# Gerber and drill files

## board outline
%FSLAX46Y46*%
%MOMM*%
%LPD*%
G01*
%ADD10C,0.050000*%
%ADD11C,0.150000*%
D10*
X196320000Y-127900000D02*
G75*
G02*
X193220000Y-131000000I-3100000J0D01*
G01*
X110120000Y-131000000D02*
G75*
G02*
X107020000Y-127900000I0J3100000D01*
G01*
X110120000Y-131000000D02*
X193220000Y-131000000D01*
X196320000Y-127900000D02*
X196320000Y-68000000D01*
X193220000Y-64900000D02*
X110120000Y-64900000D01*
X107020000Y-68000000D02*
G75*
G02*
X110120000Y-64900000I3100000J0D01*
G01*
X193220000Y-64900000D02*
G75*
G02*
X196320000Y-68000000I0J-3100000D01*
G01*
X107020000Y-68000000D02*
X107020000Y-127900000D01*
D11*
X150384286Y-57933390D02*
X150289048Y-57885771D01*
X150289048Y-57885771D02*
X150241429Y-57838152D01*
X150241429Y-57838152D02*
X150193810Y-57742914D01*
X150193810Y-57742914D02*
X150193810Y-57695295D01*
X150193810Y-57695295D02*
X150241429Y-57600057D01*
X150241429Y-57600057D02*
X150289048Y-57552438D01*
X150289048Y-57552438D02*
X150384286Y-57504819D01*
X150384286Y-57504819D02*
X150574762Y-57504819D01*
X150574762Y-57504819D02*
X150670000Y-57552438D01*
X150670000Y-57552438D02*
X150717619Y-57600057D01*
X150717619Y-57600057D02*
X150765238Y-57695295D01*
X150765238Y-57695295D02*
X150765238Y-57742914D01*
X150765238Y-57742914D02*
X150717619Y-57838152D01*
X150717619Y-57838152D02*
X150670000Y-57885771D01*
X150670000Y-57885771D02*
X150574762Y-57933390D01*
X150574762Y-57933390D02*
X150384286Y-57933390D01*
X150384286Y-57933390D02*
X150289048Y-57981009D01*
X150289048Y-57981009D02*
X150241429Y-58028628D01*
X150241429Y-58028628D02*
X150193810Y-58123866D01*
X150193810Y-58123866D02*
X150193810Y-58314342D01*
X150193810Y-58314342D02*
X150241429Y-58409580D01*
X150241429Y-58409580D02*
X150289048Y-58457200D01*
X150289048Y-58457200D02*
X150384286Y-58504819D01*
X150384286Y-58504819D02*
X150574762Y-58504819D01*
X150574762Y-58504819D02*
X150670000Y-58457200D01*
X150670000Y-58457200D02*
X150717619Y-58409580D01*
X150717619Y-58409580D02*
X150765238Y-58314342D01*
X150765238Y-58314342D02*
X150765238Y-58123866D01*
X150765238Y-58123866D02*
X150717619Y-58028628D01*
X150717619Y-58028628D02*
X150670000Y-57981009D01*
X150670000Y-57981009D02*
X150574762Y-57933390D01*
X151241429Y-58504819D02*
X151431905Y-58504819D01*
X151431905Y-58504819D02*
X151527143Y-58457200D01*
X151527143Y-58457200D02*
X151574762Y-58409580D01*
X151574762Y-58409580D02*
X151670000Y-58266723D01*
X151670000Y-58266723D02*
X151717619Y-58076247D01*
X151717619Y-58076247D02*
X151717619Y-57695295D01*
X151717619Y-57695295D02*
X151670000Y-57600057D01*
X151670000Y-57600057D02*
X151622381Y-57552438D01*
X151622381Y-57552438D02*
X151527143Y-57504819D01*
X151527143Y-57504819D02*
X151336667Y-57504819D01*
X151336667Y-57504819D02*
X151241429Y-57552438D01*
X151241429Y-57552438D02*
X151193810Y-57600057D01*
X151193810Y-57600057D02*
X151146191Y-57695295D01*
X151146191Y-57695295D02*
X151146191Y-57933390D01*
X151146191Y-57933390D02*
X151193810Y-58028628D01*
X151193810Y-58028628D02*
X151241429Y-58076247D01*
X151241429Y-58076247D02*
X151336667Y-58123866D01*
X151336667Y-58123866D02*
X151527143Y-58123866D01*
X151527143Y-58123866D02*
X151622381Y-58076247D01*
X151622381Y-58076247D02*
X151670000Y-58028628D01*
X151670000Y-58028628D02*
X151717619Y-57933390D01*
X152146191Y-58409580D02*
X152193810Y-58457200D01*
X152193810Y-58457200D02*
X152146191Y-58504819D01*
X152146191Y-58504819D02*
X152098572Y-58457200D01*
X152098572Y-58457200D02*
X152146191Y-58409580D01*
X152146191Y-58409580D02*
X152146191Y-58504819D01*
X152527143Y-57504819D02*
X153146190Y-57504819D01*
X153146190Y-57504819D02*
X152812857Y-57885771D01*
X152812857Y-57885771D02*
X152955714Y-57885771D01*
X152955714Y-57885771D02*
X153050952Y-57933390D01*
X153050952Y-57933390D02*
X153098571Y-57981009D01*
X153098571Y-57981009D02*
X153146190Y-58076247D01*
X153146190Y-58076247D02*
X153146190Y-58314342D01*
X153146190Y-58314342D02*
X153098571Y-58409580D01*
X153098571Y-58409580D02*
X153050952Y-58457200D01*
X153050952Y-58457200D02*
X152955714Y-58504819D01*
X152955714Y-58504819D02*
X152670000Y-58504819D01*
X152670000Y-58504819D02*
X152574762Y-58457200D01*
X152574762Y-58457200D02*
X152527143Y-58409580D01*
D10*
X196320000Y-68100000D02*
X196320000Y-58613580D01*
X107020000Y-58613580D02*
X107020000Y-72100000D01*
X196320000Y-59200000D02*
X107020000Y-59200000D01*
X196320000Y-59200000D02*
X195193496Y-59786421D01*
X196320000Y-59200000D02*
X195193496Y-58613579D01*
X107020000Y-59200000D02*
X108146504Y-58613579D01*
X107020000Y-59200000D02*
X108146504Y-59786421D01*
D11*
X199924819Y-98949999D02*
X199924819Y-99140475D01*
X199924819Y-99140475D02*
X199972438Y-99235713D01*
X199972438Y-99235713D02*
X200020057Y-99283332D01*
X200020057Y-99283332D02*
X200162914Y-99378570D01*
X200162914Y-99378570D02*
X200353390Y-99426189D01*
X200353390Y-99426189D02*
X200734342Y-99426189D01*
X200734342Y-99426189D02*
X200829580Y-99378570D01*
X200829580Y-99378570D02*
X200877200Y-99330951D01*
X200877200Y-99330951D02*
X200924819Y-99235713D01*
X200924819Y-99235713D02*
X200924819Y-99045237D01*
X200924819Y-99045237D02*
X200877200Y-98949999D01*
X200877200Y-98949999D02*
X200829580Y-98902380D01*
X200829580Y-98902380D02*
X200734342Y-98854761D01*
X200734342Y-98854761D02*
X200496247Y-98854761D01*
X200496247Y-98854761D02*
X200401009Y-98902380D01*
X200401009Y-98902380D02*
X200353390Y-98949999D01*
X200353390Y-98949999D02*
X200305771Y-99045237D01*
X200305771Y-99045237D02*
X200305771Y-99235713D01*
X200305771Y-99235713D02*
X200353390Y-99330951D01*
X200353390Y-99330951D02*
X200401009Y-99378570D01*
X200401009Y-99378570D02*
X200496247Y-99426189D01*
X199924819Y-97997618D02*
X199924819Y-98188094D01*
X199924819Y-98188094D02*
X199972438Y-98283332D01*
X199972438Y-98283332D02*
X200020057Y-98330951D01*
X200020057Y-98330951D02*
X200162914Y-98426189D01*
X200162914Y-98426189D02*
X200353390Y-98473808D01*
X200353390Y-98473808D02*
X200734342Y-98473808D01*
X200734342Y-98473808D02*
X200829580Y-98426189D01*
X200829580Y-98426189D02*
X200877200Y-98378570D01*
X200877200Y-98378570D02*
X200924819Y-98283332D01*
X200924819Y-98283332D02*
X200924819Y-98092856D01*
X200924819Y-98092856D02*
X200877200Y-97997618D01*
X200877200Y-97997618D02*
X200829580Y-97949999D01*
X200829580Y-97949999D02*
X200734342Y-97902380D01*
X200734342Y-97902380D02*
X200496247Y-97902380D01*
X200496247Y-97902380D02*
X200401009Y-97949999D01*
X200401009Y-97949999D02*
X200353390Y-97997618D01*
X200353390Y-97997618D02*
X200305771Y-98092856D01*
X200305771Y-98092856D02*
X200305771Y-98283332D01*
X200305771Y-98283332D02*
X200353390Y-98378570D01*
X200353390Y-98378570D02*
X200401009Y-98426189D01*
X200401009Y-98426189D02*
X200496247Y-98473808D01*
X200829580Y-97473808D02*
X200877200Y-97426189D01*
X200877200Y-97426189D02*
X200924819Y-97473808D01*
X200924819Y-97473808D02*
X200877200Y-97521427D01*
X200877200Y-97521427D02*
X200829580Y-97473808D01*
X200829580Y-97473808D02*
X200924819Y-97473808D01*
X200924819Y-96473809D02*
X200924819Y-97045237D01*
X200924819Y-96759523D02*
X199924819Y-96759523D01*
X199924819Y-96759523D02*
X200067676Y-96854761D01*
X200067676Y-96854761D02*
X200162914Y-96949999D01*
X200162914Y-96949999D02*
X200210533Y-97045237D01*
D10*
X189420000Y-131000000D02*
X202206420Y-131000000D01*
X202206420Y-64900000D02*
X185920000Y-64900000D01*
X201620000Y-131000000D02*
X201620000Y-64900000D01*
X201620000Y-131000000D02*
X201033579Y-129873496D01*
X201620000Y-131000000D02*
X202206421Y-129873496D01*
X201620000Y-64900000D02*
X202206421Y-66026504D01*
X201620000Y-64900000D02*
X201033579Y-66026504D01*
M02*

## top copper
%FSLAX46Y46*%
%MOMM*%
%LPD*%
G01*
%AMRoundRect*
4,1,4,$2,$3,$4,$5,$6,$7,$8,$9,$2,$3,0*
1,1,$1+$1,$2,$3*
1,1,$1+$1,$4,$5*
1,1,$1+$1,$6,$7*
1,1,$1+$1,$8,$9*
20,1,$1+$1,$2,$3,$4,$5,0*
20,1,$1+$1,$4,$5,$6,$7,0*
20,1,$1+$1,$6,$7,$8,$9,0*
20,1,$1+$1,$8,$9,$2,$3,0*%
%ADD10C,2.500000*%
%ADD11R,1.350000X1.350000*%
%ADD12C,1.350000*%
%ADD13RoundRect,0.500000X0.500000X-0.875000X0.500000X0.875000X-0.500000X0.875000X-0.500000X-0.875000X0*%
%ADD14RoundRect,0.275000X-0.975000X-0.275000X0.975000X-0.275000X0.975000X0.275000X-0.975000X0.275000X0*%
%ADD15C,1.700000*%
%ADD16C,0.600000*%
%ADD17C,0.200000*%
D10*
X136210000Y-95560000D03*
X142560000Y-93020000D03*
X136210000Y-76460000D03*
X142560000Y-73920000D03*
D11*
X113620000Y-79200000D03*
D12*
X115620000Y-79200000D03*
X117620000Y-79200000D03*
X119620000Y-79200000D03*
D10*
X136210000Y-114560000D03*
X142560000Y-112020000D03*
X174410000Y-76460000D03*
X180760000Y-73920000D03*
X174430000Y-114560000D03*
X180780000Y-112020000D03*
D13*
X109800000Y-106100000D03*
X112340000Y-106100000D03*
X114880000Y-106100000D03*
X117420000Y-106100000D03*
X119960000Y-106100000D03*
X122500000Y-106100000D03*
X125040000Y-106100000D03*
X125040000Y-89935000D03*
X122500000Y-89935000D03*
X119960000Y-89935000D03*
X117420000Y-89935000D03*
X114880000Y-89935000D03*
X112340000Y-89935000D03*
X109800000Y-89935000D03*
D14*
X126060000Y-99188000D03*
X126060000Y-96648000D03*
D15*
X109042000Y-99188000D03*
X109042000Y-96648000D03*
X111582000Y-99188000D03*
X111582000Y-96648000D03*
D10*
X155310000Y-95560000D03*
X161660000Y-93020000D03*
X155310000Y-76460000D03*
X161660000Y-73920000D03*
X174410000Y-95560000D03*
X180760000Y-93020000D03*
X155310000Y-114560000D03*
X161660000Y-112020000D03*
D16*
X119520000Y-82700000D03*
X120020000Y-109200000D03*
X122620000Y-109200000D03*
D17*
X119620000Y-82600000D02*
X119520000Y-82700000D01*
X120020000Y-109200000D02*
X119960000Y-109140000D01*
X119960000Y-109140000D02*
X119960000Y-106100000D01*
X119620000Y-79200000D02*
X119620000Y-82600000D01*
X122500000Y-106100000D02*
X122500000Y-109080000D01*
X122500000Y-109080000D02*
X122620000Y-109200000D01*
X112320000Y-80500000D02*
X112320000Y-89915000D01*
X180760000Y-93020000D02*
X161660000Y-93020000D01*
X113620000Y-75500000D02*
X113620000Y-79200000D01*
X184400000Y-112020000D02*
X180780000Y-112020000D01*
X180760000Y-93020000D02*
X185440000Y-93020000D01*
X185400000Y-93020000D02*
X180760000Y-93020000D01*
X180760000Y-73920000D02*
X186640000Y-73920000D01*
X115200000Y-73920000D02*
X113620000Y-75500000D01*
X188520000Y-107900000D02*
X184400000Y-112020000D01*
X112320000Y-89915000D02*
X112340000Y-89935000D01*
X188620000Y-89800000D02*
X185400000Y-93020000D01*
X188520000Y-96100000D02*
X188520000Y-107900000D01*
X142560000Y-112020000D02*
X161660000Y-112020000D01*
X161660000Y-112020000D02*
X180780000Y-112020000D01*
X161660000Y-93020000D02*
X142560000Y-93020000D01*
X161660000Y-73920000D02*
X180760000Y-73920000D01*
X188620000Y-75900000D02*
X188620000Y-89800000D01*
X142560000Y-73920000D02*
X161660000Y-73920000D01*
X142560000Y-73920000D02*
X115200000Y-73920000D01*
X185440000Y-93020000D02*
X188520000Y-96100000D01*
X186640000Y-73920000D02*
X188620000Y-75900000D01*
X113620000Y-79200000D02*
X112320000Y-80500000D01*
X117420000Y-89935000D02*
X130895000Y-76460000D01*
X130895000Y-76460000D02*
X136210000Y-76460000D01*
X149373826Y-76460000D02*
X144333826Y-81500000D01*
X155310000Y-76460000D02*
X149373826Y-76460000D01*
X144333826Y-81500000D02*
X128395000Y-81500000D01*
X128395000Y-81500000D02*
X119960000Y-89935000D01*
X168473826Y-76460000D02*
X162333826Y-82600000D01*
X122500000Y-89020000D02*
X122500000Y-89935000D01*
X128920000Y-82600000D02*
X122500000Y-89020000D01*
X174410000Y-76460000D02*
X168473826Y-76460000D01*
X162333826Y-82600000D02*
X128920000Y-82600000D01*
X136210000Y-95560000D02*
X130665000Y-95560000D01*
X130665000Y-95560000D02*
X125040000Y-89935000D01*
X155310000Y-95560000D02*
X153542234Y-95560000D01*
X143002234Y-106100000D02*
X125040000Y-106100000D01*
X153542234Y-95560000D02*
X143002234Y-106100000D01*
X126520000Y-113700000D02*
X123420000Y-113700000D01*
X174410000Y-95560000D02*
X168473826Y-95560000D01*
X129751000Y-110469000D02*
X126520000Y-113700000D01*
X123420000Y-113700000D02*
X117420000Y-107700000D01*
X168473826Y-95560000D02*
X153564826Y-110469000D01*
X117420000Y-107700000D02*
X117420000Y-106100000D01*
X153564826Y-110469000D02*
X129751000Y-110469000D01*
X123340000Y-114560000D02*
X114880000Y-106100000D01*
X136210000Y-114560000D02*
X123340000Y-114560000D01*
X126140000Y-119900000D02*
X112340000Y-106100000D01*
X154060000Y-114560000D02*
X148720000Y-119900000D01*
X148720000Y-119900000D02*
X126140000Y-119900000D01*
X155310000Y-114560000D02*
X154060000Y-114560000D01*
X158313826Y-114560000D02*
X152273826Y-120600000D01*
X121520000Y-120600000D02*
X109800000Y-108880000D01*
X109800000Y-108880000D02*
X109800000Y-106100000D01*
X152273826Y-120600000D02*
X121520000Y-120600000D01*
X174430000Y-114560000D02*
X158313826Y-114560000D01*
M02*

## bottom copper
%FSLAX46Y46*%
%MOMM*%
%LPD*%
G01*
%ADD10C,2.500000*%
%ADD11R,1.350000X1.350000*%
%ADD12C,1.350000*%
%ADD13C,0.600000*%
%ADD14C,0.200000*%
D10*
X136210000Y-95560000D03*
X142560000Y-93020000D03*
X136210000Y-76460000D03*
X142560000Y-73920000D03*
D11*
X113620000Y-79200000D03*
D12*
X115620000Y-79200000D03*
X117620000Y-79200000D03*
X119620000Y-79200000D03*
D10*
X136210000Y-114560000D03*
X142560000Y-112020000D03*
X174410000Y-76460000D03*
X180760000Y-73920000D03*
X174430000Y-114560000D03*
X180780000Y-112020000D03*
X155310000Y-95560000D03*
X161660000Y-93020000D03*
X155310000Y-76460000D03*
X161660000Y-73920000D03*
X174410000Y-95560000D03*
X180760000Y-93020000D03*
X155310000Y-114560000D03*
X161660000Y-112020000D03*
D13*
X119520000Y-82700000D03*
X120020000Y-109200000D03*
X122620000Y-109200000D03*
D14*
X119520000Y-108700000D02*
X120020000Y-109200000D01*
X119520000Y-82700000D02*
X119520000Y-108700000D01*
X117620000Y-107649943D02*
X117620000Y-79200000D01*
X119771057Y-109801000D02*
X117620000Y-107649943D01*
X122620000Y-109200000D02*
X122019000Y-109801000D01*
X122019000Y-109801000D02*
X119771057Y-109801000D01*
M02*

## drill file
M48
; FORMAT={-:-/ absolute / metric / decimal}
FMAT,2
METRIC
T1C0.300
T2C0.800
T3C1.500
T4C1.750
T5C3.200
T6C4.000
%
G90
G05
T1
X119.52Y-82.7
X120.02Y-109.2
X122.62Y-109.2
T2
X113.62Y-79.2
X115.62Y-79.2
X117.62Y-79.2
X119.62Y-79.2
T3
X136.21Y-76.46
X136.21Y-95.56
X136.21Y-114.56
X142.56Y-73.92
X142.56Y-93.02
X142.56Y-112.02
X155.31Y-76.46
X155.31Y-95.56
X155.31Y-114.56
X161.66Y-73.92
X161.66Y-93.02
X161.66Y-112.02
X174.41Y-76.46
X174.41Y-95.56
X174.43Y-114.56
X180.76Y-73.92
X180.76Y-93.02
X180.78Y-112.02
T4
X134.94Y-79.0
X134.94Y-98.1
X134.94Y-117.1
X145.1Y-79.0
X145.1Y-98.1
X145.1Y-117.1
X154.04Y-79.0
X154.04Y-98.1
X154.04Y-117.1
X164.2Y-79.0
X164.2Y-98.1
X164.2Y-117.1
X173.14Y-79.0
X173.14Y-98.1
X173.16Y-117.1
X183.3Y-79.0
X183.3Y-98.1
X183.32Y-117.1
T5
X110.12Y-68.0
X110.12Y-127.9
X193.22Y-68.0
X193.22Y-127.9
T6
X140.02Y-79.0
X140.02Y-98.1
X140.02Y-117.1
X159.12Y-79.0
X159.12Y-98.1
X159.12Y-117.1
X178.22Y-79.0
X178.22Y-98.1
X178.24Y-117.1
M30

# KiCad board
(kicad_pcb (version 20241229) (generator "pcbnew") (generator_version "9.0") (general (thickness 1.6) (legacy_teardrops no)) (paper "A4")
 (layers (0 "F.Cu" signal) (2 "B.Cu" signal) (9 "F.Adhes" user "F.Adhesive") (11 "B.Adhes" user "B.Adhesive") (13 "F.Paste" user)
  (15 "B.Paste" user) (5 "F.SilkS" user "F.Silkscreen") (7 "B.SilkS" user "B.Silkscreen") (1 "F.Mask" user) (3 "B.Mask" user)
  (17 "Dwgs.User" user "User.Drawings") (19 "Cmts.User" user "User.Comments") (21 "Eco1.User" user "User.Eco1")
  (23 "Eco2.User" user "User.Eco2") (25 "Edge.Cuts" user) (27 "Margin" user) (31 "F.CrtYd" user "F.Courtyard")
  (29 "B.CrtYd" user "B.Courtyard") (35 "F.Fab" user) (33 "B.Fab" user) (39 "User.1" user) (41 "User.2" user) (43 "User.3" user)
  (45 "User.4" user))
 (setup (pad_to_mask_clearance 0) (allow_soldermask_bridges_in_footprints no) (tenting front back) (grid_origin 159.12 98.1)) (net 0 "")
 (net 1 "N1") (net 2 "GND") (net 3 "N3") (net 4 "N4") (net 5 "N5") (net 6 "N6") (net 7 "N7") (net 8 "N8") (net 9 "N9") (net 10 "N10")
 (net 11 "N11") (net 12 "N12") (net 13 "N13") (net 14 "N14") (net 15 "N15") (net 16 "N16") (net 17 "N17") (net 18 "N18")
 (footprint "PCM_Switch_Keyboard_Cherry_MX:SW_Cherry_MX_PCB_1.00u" (layer "F.Cu") (at 140.02 98.1)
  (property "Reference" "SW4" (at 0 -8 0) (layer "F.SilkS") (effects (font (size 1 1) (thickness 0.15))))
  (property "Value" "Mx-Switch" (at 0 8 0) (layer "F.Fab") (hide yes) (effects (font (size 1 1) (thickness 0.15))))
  (pad "" np_thru_hole circle (at -5.08 0) (size 1.75 1.75) (drill 1.75) (layers "*.Cu" "*.Mask"))
  (pad "" np_thru_hole circle (at 0 0) (size 4 4) (drill 4) (layers "*.Cu" "*.Mask"))
  (pad "" np_thru_hole circle (at 5.08 0) (size 1.75 1.75) (drill 1.75) (layers "*.Cu" "*.Mask"))
  (pad "1" thru_hole circle (at -3.81 -2.54) (size 2.5 2.5) (drill 1.5) (layers "*.Cu" "*.Mask") (remove_unused_layers no) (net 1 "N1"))
  (pad "2" thru_hole circle (at 2.54 -5.08) (size 2.5 2.5) (drill 1.5) (layers "*.Cu" "*.Mask") (remove_unused_layers no) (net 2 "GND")))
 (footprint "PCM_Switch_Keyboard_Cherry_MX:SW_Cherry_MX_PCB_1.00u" (layer "F.Cu") (at 140.02 79)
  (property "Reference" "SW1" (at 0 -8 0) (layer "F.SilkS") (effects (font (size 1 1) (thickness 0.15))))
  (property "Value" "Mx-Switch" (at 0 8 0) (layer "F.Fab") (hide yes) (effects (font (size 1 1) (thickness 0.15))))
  (pad "" np_thru_hole circle (at -5.08 0) (size 1.75 1.75) (drill 1.75) (layers "*.Cu" "*.Mask"))
  (pad "" np_thru_hole circle (at 0 0) (size 4 4) (drill 4) (layers "*.Cu" "*.Mask"))
  (pad "" np_thru_hole circle (at 5.08 0) (size 1.75 1.75) (drill 1.75) (layers "*.Cu" "*.Mask"))
  (pad "1" thru_hole circle (at -3.81 -2.54) (size 2.5 2.5) (drill 1.5) (layers "*.Cu" "*.Mask") (remove_unused_layers no) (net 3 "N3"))
  (pad "2" thru_hole circle (at 2.54 -5.08) (size 2.5 2.5) (drill 1.5) (layers "*.Cu" "*.Mask") (remove_unused_layers no) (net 2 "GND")))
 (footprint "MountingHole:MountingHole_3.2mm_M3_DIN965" (layer "F.Cu") (at 193.22 68)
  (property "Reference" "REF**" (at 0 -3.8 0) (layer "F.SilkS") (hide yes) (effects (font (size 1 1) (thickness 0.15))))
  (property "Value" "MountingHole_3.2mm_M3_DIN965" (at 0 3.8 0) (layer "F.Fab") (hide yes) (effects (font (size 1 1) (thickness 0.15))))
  (pad "" np_thru_hole circle (at 0 0) (size 3.2 3.2) (drill 3.2) (layers "*.Cu" "*.Mask")))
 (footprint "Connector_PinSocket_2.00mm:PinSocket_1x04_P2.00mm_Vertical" (layer "F.Cu") (at 113.62 79.2 90)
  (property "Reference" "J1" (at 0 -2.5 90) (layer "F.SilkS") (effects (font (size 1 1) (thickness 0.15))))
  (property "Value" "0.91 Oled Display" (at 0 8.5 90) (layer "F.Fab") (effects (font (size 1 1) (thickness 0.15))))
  (pad "1" thru_hole rect (at 0 0 90) (size 1.35 1.35) (drill 0.8) (layers "*.Cu" "*.Mask") (remove_unused_layers no) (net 2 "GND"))
  (pad "2" thru_hole circle (at 0 2 90) (size 1.35 1.35) (drill 0.8) (layers "*.Cu" "*.Mask") (remove_unused_layers no) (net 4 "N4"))
  (pad "3" thru_hole circle (at 0 4 90) (size 1.35 1.35) (drill 0.8) (layers "*.Cu" "*.Mask") (remove_unused_layers no) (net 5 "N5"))
  (pad "4" thru_hole circle (at 0 6 90) (size 1.35 1.35) (drill 0.8) (layers "*.Cu" "*.Mask") (remove_unused_layers no) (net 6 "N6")))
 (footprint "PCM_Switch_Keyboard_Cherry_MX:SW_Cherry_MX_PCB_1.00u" (layer "F.Cu") (at 140.02 117.1)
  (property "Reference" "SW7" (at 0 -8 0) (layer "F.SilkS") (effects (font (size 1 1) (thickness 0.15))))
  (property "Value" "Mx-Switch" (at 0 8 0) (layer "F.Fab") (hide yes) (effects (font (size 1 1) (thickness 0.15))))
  (pad "" np_thru_hole circle (at -5.08 0) (size 1.75 1.75) (drill 1.75) (layers "*.Cu" "*.Mask"))
  (pad "" np_thru_hole circle (at 0 0) (size 4 4) (drill 4) (layers "*.Cu" "*.Mask"))
  (pad "" np_thru_hole circle (at 5.08 0) (size 1.75 1.75) (drill 1.75) (layers "*.Cu" "*.Mask"))
  (pad "1" thru_hole circle (at -3.81 -2.54) (size 2.5 2.5) (drill 1.5) (layers "*.Cu" "*.Mask") (remove_unused_layers no) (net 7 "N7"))
  (pad "2" thru_hole circle (at 2.54 -5.08) (size 2.5 2.5) (drill 1.5) (layers "*.Cu" "*.Mask") (remove_unused_layers no) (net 2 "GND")))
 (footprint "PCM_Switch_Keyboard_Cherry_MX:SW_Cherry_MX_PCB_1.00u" (layer "F.Cu") (at 178.22 79)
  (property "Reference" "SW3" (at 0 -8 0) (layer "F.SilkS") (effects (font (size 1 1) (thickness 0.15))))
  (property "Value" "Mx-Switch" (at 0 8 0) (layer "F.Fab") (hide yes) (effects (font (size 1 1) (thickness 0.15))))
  (pad "" np_thru_hole circle (at -5.08 0) (size 1.75 1.75) (drill 1.75) (layers "*.Cu" "*.Mask"))
  (pad "" np_thru_hole circle (at 0 0) (size 4 4) (drill 4) (layers "*.Cu" "*.Mask"))
  (pad "" np_thru_hole circle (at 5.08 0) (size 1.75 1.75) (drill 1.75) (layers "*.Cu" "*.Mask"))
  (pad "1" thru_hole circle (at -3.81 -2.54) (size 2.5 2.5) (drill 1.5) (layers "*.Cu" "*.Mask") (remove_unused_layers no) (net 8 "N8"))
  (pad "2" thru_hole circle (at 2.54 -5.08) (size 2.5 2.5) (drill 1.5) (layers "*.Cu" "*.Mask") (remove_unused_layers no) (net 2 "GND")))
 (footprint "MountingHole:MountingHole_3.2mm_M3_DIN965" (layer "F.Cu") (at 110.12 68)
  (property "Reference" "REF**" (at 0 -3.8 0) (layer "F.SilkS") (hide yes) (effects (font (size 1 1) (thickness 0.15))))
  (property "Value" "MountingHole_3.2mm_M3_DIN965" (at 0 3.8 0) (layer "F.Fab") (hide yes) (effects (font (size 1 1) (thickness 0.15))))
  (pad "" np_thru_hole circle (at 0 0) (size 3.2 3.2) (drill 3.2) (layers "*.Cu" "*.Mask")))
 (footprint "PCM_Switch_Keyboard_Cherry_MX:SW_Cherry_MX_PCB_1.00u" (layer "F.Cu") (at 178.24 117.1)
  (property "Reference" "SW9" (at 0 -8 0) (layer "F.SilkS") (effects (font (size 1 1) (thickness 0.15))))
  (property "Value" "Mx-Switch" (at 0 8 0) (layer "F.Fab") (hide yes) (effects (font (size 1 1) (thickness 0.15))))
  (pad "" np_thru_hole circle (at -5.08 0) (size 1.75 1.75) (drill 1.75) (layers "*.Cu" "*.Mask"))
  (pad "" np_thru_hole circle (at 0 0) (size 4 4) (drill 4) (layers "*.Cu" "*.Mask"))
  (pad "" np_thru_hole circle (at 5.08 0) (size 1.75 1.75) (drill 1.75) (layers "*.Cu" "*.Mask"))
  (pad "1" thru_hole circle (at -3.81 -2.54) (size 2.5 2.5) (drill 1.5) (layers "*.Cu" "*.Mask") (remove_unused_layers no) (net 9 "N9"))
  (pad "2" thru_hole circle (at 2.54 -5.08) (size 2.5 2.5) (drill 1.5) (layers "*.Cu" "*.Mask") (remove_unused_layers no) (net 2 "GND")))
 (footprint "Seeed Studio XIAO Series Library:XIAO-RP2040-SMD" (layer "F.Cu") (at 117.42 98.1 90)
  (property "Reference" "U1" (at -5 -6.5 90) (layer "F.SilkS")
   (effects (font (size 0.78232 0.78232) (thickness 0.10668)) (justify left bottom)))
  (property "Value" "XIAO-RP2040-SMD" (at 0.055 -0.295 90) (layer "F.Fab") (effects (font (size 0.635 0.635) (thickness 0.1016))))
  (pad "1" smd roundrect (at -8 -7.62 90) (size 2.75 2) (layers "F.Cu" "F.Mask" "F.Paste") (roundrect_rratio 0.25) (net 9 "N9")
   (solder_mask_margin 0.0508) (thermal_bridge_angle 45))
  (pad "2" smd roundrect (at -8 -5.08 90) (size 2.75 2) (layers "F.Cu" "F.Mask" "F.Paste") (roundrect_rratio 0.25) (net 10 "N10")
   (solder_mask_margin 0.0508) (thermal_bridge_angle 45))
  (pad "3" smd roundrect (at -8 -2.54 90) (size 2.75 2) (layers "F.Cu" "F.Mask" "F.Paste") (roundrect_rratio 0.25) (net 7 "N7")
   (solder_mask_margin 0.0508) (thermal_bridge_angle 45))
  (pad "4" smd roundrect (at -8 0 90) (size 2.75 2) (layers "F.Cu" "F.Mask" "F.Paste") (roundrect_rratio 0.25) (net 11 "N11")
   (solder_mask_margin 0.0508) (thermal_bridge_angle 45))
  (pad "5" smd roundrect (at -8 2.54 90) (size 2.75 2) (layers "F.Cu" "F.Mask" "F.Paste") (roundrect_rratio 0.25) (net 6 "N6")
   (solder_mask_margin 0.0508) (thermal_bridge_angle 45))
  (pad "6" smd roundrect (at -8 5.08 90) (size 2.75 2) (layers "F.Cu" "F.Mask" "F.Paste") (roundrect_rratio 0.25) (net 5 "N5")
   (solder_mask_margin 0.0508) (thermal_bridge_angle 45))
  (pad "7" smd roundrect (at -8 7.62 90) (size 2.75 2) (layers "F.Cu" "F.Mask" "F.Paste") (roundrect_rratio 0.25) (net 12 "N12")
   (solder_mask_margin 0.0508) (thermal_bridge_angle 45))
  (pad "8" smd roundrect (at 8.165 7.62 90) (size 2.75 2) (layers "F.Cu" "F.Mask" "F.Paste") (roundrect_rratio 0.25) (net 1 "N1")
   (solder_mask_margin 0.0508) (thermal_bridge_angle 45))
  (pad "9" smd roundrect (at 8.165 5.08 90) (size 2.75 2) (layers "F.Cu" "F.Mask" "F.Paste") (roundrect_rratio 0.25) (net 8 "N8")
   (solder_mask_margin 0.0508) (thermal_bridge_angle 45))
  (pad "10" smd roundrect (at 8.165 2.54 90) (size 2.75 2) (layers "F.Cu" "F.Mask" "F.Paste") (roundrect_rratio 0.25) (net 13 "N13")
   (solder_mask_margin 0.0508) (thermal_bridge_angle 45))
  (pad "11" smd roundrect (at 8.165 0 90) (size 2.75 2) (layers "F.Cu" "F.Mask" "F.Paste") (roundrect_rratio 0.25) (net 3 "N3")
   (solder_mask_margin 0.0508) (thermal_bridge_angle 45))
  (pad "12" smd roundrect (at 8.165 -2.54 90) (size 2.75 2) (layers "F.Cu" "F.Mask" "F.Paste") (roundrect_rratio 0.25) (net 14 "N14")
   (solder_mask_margin 0.0508) (thermal_bridge_angle 45))
  (pad "13" smd roundrect (at 8.165 -5.08 90) (size 2.75 2) (layers "F.Cu" "F.Mask" "F.Paste") (roundrect_rratio 0.25) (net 2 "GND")
   (solder_mask_margin 0.0508) (thermal_bridge_angle 45))
  (pad "14" smd roundrect (at 8.165 -7.62 90) (size 2.75 2) (layers "F.Cu" "F.Mask" "F.Paste") (roundrect_rratio 0.25) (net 4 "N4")
   (solder_mask_margin 0.0508) (thermal_bridge_angle 45))
  (pad "15" smd roundrect (at -1.088 8.64) (size 2.5 1.1) (layers "F.Cu" "F.Mask" "F.Paste") (roundrect_rratio 0.25) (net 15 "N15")
   (thermal_bridge_angle 45))
  (pad "16" smd roundrect (at 1.452 8.64) (size 2.5 1.1) (layers "F.Cu" "F.Mask" "F.Paste") (roundrect_rratio 0.25) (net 2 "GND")
   (thermal_bridge_angle 45))
  (pad "17" smd circle (at -1.088 -8.378 90) (size 1.7 1.7) (layers "F.Cu" "F.Mask" "F.Paste") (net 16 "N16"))
  (pad "18" smd circle (at 1.452 -8.378 90) (size 1.7 1.7) (layers "F.Cu" "F.Mask" "F.Paste") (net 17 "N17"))
  (pad "19" smd circle (at -1.088 -5.838 90) (size 1.7 1.7) (layers "F.Cu" "F.Mask" "F.Paste") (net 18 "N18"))
  (pad "20" smd circle (at 1.452 -5.838 90) (size 1.7 1.7) (layers "F.Cu" "F.Mask" "F.Paste") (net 2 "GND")))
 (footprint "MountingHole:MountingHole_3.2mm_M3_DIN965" (layer "F.Cu") (at 110.12 127.9)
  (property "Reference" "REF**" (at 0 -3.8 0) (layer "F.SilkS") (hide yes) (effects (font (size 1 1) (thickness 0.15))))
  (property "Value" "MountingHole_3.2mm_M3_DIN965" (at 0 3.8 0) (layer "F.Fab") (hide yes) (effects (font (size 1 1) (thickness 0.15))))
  (pad "" np_thru_hole circle (at 0 0) (size 3.2 3.2) (drill 3.2) (layers "*.Cu" "*.Mask")))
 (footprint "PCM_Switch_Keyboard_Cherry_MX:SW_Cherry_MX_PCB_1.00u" (layer "F.Cu") (at 159.12 98.1)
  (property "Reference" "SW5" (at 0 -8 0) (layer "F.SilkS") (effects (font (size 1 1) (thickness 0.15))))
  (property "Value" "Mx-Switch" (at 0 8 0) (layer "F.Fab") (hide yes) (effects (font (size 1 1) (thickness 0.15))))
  (pad "" np_thru_hole circle (at -5.08 0) (size 1.75 1.75) (drill 1.75) (layers "*.Cu" "*.Mask"))
  (pad "" np_thru_hole circle (at 0 0) (size 4 4) (drill 4) (layers "*.Cu" "*.Mask"))
  (pad "" np_thru_hole circle (at 5.08 0) (size 1.75 1.75) (drill 1.75) (layers "*.Cu" "*.Mask"))
  (pad "1" thru_hole circle (at -3.81 -2.54) (size 2.5 2.5) (drill 1.5) (layers "*.Cu" "*.Mask") (remove_unused_layers no) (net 12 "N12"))
  (pad "2" thru_hole circle (at 2.54 -5.08) (size 2.5 2.5) (drill 1.5) (layers "*.Cu" "*.Mask") (remove_unused_layers no) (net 2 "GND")))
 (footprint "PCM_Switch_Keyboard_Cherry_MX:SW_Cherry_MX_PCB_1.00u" (layer "F.Cu") (at 159.12 79)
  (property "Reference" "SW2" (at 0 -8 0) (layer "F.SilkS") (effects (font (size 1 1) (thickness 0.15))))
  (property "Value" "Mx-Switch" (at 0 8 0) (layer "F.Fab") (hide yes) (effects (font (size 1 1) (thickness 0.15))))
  (pad "" np_thru_hole circle (at -5.08 0) (size 1.75 1.75) (drill 1.75) (layers "*.Cu" "*.Mask"))
  (pad "" np_thru_hole circle (at 0 0) (size 4 4) (drill 4) (layers "*.Cu" "*.Mask"))
  (pad "" np_thru_hole circle (at 5.08 0) (size 1.75 1.75) (drill 1.75) (layers "*.Cu" "*.Mask"))
  (pad "1" thru_hole circle (at -3.81 -2.54) (size 2.5 2.5) (drill 1.5) (layers "*.Cu" "*.Mask") (remove_unused_layers no) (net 13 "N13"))
  (pad "2" thru_hole circle (at 2.54 -5.08) (size 2.5 2.5) (drill 1.5) (layers "*.Cu" "*.Mask") (remove_unused_layers no) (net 2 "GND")))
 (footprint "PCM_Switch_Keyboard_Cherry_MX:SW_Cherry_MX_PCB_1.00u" (layer "F.Cu") (at 178.22 98.1)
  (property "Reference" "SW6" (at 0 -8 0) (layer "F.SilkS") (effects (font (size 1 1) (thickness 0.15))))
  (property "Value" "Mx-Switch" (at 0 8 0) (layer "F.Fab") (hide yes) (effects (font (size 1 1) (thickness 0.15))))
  (pad "" np_thru_hole circle (at -5.08 0) (size 1.75 1.75) (drill 1.75) (layers "*.Cu" "*.Mask"))
  (pad "" np_thru_hole circle (at 0 0) (size 4 4) (drill 4) (layers "*.Cu" "*.Mask"))
  (pad "" np_thru_hole circle (at 5.08 0) (size 1.75 1.75) (drill 1.75) (layers "*.Cu" "*.Mask"))
  (pad "1" thru_hole circle (at -3.81 -2.54) (size 2.5 2.5) (drill 1.5) (layers "*.Cu" "*.Mask") (remove_unused_layers no) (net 11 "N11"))
  (pad "2" thru_hole circle (at 2.54 -5.08) (size 2.5 2.5) (drill 1.5) (layers "*.Cu" "*.Mask") (remove_unused_layers no) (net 2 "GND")))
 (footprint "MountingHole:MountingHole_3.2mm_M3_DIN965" (layer "F.Cu") (at 193.22 127.9)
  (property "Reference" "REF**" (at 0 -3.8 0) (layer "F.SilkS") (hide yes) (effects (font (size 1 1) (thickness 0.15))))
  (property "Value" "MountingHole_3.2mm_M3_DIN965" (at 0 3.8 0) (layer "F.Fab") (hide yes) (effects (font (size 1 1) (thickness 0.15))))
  (pad "" np_thru_hole circle (at 0 0) (size 3.2 3.2) (drill 3.2) (layers "*.Cu" "*.Mask")))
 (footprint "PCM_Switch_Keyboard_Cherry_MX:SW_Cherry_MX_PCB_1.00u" (layer "F.Cu") (at 159.12 117.1)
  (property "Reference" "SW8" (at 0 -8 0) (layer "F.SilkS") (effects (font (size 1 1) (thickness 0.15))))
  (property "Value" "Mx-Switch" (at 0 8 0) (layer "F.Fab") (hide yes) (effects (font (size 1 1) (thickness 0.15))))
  (pad "" np_thru_hole circle (at -5.08 0) (size 1.75 1.75) (drill 1.75) (layers "*.Cu" "*.Mask"))
  (pad "" np_thru_hole circle (at 0 0) (size 4 4) (drill 4) (layers "*.Cu" "*.Mask"))
  (pad "" np_thru_hole circle (at 5.08 0) (size 1.75 1.75) (drill 1.75) (layers "*.Cu" "*.Mask"))
  (pad "1" thru_hole circle (at -3.81 -2.54) (size 2.5 2.5) (drill 1.5) (layers "*.Cu" "*.Mask") (remove_unused_layers no) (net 10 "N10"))
  (pad "2" thru_hole circle (at 2.54 -5.08) (size 2.5 2.5) (drill 1.5) (layers "*.Cu" "*.Mask") (remove_unused_layers no) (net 2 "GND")))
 (gr_arc (start 196.32 127.9) (mid 195.412031 130.092031) (end 193.22 131) (stroke (width 0.05) (type default)) (layer "Edge.Cuts"))
 (gr_arc (start 110.12 131) (mid 107.927969 130.092031) (end 107.02 127.9) (stroke (width 0.05) (type default)) (layer "Edge.Cuts"))
 (gr_line (start 110.12 131) (end 193.22 131) (stroke (width 0.05) (type default)) (layer "Edge.Cuts"))
 (gr_line (start 196.32 127.9) (end 196.32 68) (stroke (width 0.05) (type default)) (layer "Edge.Cuts"))
 (gr_line (start 193.22 64.9) (end 110.12 64.9) (stroke (width 0.05) (type default)) (layer "Edge.Cuts"))
 (gr_arc (start 107.02 68) (mid 107.927969 65.807969) (end 110.12 64.9) (stroke (width 0.05) (type solid)) (layer "Edge.Cuts"))
 (gr_arc (start 193.22 64.9) (mid 195.412031 65.807969) (end 196.32 68) (stroke (width 0.05) (type default)) (layer "Edge.Cuts"))
 (gr_line (start 107.02 68) (end 107.02 127.9) (stroke (width 0.05) (type default)) (layer "Edge.Cuts"))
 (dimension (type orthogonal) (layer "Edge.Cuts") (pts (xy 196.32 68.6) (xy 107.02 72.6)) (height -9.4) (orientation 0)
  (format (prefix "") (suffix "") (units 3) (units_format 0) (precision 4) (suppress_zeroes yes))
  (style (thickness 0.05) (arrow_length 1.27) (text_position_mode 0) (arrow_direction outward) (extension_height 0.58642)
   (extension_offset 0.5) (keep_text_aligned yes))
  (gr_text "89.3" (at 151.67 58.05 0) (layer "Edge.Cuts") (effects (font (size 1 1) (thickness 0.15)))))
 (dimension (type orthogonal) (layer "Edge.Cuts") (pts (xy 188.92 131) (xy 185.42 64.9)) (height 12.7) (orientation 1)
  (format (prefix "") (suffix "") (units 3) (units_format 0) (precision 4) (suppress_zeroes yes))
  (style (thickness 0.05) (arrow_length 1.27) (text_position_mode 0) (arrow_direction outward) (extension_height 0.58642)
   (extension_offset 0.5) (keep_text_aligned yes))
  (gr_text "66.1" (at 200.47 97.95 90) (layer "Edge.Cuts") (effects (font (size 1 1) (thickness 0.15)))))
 (segment (start 119.62 82.6) (end 119.52 82.7) (width 0.2) (layer "F.Cu") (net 6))
 (segment (start 120.02 109.2) (end 119.96 109.14) (width 0.2) (layer "F.Cu") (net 6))
 (segment (start 119.96 109.14) (end 119.96 106.1) (width 0.2) (layer "F.Cu") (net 6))
 (segment (start 119.62 79.2) (end 119.62 82.6) (width 0.2) (layer "F.Cu") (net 6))
 (via (at 119.52 82.7) (size 0.6) (drill 0.3) (layers "F.Cu" "B.Cu") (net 6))
 (via (at 120.02 109.2) (size 0.6) (drill 0.3) (layers "F.Cu" "B.Cu") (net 6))
 (segment (start 119.52 108.7) (end 120.02 109.2) (width 0.2) (layer "B.Cu") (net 6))
 (segment (start 119.52 82.7) (end 119.52 108.7) (width 0.2) (layer "B.Cu") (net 6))
 (segment (start 122.5 106.1) (end 122.5 109.08) (width 0.2) (layer "F.Cu") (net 5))
 (segment (start 122.5 109.08) (end 122.62 109.2) (width 0.2) (layer "F.Cu") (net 5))
 (via (at 122.62 109.2) (size 0.6) (drill 0.3) (layers "F.Cu" "B.Cu") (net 5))
 (segment (start 117.62 107.649943) (end 117.62 79.2) (width 0.2) (layer "B.Cu") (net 5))
 (segment (start 119.771057 109.801) (end 117.62 107.649943) (width 0.2) (layer "B.Cu") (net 5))
 (segment (start 122.62 109.2) (end 122.019 109.801) (width 0.2) (layer "B.Cu") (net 5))
 (segment (start 122.019 109.801) (end 119.771057 109.801) (width 0.2) (layer "B.Cu") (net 5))
 (segment (start 112.32 80.5) (end 112.32 89.915) (width 0.2) (layer "F.Cu") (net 2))
 (segment (start 180.76 93.02) (end 161.66 93.02) (width 0.2) (layer "F.Cu") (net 2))
 (segment (start 113.62 75.5) (end 113.62 79.2) (width 0.2) (layer "F.Cu") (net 2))
 (segment (start 184.4 112.02) (end 180.78 112.02) (width 0.2) (layer "F.Cu") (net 2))
 (segment (start 180.76 93.02) (end 185.44 93.02) (width 0.2) (layer "F.Cu") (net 2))
 (segment (start 185.4 93.02) (end 180.76 93.02) (width 0.2) (layer "F.Cu") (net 2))
 (segment (start 180.76 73.92) (end 186.64 73.92) (width 0.2) (layer "F.Cu") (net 2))
 (segment (start 115.2 73.92) (end 113.62 75.5) (width 0.2) (layer "F.Cu") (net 2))
 (segment (start 188.52 107.9) (end 184.4 112.02) (width 0.2) (layer "F.Cu") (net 2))
 (segment (start 112.32 89.915) (end 112.34 89.935) (width 0.2) (layer "F.Cu") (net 2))
 (segment (start 188.62 89.8) (end 185.4 93.02) (width 0.2) (layer "F.Cu") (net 2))
 (segment (start 188.52 96.1) (end 188.52 107.9) (width 0.2) (layer "F.Cu") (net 2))
 (segment (start 142.56 112.02) (end 161.66 112.02) (width 0.2) (layer "F.Cu") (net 2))
 (segment (start 161.66 112.02) (end 180.78 112.02) (width 0.2) (layer "F.Cu") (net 2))
 (segment (start 161.66 93.02) (end 142.56 93.02) (width 0.2) (layer "F.Cu") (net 2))
 (segment (start 161.66 73.92) (end 180.76 73.92) (width 0.2) (layer "F.Cu") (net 2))
 (segment (start 188.62 75.9) (end 188.62 89.8) (width 0.2) (layer "F.Cu") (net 2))
 (segment (start 142.56 73.92) (end 161.66 73.92) (width 0.2) (layer "F.Cu") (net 2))
 (segment (start 142.56 73.92) (end 115.2 73.92) (width 0.2) (layer "F.Cu") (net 2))
 (segment (start 185.44 93.02) (end 188.52 96.1) (width 0.2) (layer "F.Cu") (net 2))
 (segment (start 186.64 73.92) (end 188.62 75.9) (width 0.2) (layer "F.Cu") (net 2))
 (segment (start 113.62 79.2) (end 112.32 80.5) (width 0.2) (layer "F.Cu") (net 2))
 (segment (start 117.42 89.935) (end 130.895 76.46) (width 0.2) (layer "F.Cu") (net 3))
 (segment (start 130.895 76.46) (end 136.21 76.46) (width 0.2) (layer "F.Cu") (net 3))
 (segment (start 149.373826 76.46) (end 144.333826 81.5) (width 0.2) (layer "F.Cu") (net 13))
 (segment (start 155.31 76.46) (end 149.373826 76.46) (width 0.2) (layer "F.Cu") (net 13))
 (segment (start 144.333826 81.5) (end 128.395 81.5) (width 0.2) (layer "F.Cu") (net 13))
 (segment (start 128.395 81.5) (end 119.96 89.935) (width 0.2) (layer "F.Cu") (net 13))
 (segment (start 168.473826 76.46) (end 162.333826 82.6) (width 0.2) (layer "F.Cu") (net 8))
 (segment (start 122.5 89.02) (end 122.5 89.935) (width 0.2) (layer "F.Cu") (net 8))
 (segment (start 128.92 82.6) (end 122.5 89.02) (width 0.2) (layer "F.Cu") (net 8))
 (segment (start 174.41 76.46) (end 168.473826 76.46) (width 0.2) (layer "F.Cu") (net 8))
 (segment (start 162.333826 82.6) (end 128.92 82.6) (width 0.2) (layer "F.Cu") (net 8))
 (segment (start 136.21 95.56) (end 130.665 95.56) (width 0.2) (layer "F.Cu") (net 1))
 (segment (start 130.665 95.56) (end 125.04 89.935) (width 0.2) (layer "F.Cu") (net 1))
 (segment (start 155.31 95.56) (end 153.542234 95.56) (width 0.2) (layer "F.Cu") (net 12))
 (segment (start 143.002234 106.1) (end 125.04 106.1) (width 0.2) (layer "F.Cu") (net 12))
 (segment (start 153.542234 95.56) (end 143.002234 106.1) (width 0.2) (layer "F.Cu") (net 12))
 (segment (start 126.52 113.7) (end 123.42 113.7) (width 0.2) (layer "F.Cu") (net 11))
 (segment (start 174.41 95.56) (end 168.473826 95.56) (width 0.2) (layer "F.Cu") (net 11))
 (segment (start 129.751 110.469) (end 126.52 113.7) (width 0.2) (layer "F.Cu") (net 11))
 (segment (start 123.42 113.7) (end 117.42 107.7) (width 0.2) (layer "F.Cu") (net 11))
 (segment (start 168.473826 95.56) (end 153.564826 110.469) (width 0.2) (layer "F.Cu") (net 11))
 (segment (start 117.42 107.7) (end 117.42 106.1) (width 0.2) (layer "F.Cu") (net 11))
 (segment (start 153.564826 110.469) (end 129.751 110.469) (width 0.2) (layer "F.Cu") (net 11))
 (segment (start 123.34 114.56) (end 114.88 106.1) (width 0.2) (layer "F.Cu") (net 7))
 (segment (start 136.21 114.56) (end 123.34 114.56) (width 0.2) (layer "F.Cu") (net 7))
 (segment (start 126.14 119.9) (end 112.34 106.1) (width 0.2) (layer "F.Cu") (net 10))
 (segment (start 154.06 114.56) (end 148.72 119.9) (width 0.2) (layer "F.Cu") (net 10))
 (segment (start 148.72 119.9) (end 126.14 119.9) (width 0.2) (layer "F.Cu") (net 10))
 (segment (start 155.31 114.56) (end 154.06 114.56) (width 0.2) (layer "F.Cu") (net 10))
 (segment (start 158.313826 114.56) (end 152.273826 120.6) (width 0.2) (layer "F.Cu") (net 9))
 (segment (start 121.52 120.6) (end 109.8 108.88) (width 0.2) (layer "F.Cu") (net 9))
 (segment (start 109.8 108.88) (end 109.8 106.1) (width 0.2) (layer "F.Cu") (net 9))
 (segment (start 152.273826 120.6) (end 121.52 120.6) (width 0.2) (layer "F.Cu") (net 9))
 (segment (start 174.43 114.56) (end 158.313826 114.56) (width 0.2) (layer "F.Cu") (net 9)))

